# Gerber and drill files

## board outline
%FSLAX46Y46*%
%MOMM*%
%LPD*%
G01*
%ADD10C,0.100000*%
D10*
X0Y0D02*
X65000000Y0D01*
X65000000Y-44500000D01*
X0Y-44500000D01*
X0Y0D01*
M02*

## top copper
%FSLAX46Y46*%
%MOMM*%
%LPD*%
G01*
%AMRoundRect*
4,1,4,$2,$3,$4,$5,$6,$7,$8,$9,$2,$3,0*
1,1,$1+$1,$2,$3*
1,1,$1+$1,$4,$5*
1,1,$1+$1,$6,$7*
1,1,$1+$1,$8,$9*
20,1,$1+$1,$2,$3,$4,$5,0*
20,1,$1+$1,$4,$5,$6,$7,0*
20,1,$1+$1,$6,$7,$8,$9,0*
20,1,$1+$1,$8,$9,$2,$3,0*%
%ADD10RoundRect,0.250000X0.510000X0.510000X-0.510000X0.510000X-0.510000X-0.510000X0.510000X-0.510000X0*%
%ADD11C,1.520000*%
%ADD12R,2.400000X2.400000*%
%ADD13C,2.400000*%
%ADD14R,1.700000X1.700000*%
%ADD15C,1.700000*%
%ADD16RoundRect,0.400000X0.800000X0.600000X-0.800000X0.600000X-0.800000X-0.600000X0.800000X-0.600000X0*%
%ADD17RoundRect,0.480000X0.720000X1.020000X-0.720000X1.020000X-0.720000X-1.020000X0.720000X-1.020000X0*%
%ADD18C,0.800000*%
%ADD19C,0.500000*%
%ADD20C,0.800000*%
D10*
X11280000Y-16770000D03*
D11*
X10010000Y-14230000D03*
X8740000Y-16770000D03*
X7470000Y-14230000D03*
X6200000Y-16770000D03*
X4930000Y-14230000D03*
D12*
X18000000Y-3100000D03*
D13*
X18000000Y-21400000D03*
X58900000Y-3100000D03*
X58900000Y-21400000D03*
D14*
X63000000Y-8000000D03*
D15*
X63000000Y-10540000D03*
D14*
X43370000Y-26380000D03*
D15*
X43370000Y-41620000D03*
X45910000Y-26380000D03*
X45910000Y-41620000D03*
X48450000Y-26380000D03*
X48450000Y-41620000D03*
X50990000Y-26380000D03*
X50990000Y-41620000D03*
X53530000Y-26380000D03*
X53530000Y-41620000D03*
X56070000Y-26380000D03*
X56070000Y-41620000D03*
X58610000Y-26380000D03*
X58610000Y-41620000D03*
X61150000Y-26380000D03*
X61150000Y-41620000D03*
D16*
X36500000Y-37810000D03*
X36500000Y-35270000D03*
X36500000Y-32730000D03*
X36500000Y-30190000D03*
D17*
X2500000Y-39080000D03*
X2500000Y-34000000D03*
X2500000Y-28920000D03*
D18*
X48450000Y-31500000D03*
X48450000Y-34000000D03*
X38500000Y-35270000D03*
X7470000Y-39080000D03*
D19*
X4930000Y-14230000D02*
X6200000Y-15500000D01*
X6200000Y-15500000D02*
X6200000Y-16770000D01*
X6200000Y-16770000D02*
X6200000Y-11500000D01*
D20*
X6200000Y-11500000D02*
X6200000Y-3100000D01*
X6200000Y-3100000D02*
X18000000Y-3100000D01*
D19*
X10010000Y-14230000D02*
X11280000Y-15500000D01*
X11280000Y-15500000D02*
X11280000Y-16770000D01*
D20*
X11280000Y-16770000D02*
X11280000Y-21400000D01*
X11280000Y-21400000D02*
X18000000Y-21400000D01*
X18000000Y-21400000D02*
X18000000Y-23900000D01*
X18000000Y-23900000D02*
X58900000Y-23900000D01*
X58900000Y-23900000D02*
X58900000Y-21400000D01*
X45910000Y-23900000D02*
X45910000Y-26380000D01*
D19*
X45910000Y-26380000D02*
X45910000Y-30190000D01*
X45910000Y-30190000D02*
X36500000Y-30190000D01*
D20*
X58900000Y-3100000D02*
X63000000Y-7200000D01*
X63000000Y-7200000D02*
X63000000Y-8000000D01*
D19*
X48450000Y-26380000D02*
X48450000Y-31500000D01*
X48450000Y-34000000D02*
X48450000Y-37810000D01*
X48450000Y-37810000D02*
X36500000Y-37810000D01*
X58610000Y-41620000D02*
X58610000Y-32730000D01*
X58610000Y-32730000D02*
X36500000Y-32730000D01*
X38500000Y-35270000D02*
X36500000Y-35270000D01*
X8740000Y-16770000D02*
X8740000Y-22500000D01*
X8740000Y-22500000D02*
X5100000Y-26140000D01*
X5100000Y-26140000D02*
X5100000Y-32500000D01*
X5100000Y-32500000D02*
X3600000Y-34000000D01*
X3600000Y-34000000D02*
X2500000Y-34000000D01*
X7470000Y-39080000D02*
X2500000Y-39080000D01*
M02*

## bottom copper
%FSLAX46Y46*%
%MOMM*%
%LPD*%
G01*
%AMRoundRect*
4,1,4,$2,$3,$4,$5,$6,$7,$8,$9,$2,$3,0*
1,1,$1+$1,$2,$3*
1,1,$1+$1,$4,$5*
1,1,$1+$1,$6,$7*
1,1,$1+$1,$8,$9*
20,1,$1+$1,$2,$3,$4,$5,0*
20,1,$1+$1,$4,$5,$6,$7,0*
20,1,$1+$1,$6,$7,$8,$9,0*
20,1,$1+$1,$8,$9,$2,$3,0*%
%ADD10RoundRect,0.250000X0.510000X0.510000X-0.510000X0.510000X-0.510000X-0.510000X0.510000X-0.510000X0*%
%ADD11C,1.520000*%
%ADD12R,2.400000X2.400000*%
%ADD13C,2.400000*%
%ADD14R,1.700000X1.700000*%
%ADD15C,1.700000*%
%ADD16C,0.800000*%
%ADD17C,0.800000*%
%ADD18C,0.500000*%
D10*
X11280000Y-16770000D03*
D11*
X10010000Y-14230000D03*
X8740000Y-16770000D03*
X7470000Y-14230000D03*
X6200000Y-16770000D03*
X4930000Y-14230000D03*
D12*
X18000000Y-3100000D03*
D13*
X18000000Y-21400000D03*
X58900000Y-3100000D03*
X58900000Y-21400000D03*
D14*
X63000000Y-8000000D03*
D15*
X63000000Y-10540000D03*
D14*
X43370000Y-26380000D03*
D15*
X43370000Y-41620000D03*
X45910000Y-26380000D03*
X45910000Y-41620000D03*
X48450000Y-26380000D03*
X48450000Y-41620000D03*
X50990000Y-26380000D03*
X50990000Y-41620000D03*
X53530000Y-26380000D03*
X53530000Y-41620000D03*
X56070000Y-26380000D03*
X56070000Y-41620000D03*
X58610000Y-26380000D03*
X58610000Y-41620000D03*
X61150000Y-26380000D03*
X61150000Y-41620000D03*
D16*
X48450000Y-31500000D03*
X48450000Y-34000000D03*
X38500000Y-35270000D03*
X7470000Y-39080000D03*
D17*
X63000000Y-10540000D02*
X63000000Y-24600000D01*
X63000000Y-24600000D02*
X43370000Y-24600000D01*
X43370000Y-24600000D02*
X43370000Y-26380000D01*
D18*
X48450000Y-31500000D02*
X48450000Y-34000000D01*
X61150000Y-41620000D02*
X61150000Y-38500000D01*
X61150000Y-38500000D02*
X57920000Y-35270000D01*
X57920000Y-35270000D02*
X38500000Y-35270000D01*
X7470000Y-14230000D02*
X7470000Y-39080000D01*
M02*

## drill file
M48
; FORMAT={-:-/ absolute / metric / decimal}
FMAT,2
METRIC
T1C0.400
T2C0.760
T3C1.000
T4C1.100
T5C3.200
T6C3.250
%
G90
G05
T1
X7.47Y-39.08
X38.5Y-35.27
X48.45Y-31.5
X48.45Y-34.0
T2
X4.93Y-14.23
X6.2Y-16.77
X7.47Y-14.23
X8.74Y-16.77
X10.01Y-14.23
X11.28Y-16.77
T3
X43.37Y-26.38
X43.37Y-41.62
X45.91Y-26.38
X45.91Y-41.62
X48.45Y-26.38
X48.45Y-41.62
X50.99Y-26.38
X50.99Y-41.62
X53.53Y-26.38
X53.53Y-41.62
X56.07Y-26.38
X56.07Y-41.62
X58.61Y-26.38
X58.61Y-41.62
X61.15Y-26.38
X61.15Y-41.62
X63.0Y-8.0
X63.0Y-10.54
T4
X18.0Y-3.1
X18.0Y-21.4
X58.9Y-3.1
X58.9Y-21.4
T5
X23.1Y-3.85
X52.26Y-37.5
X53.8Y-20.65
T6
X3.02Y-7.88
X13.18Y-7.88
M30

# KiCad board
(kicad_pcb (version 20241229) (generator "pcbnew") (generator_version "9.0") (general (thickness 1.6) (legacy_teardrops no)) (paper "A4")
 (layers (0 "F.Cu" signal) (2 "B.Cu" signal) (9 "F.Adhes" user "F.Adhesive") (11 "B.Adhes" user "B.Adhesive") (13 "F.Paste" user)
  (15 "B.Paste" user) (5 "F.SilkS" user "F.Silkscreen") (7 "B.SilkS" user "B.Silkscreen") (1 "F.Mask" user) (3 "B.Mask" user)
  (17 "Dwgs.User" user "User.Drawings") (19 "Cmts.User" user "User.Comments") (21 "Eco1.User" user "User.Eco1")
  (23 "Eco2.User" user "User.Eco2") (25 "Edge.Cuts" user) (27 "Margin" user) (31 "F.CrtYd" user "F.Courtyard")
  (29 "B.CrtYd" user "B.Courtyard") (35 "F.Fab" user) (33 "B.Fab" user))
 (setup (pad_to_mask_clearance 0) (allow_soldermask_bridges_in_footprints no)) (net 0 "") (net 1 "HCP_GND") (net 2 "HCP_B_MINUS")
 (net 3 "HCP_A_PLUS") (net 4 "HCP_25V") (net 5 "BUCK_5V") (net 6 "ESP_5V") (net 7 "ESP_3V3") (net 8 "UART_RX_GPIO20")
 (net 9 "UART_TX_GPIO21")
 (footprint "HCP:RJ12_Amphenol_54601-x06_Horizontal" (layer "F.Cu") (at 11.28 16.77 180)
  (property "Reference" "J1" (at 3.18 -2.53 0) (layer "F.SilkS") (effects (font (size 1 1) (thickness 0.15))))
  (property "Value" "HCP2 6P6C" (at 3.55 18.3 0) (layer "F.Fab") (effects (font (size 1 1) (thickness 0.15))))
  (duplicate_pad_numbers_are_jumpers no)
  (pad "" np_thru_hole circle (at -1.9 8.89 180) (size 3.25 3.25) (drill 3.25) (layers "*.Cu" "*.Mask"))
  (pad "" np_thru_hole circle (at 8.26 8.89 180) (size 3.25 3.25) (drill 3.25) (layers "*.Cu" "*.Mask"))
  (pad "1" thru_hole roundrect (at 0 0 180) (size 1.52 1.52) (drill 0.76) (layers "*.Cu" "*.Mask") (remove_unused_layers no)
   (roundrect_rratio 0.1644736842) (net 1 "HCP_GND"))
  (pad "2" thru_hole circle (at 1.27 2.54 180) (size 1.52 1.52) (drill 0.76) (layers "*.Cu" "*.Mask") (remove_unused_layers no)
   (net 1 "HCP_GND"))
  (pad "3" thru_hole circle (at 2.54 0 180) (size 1.52 1.52) (drill 0.76) (layers "*.Cu" "*.Mask") (remove_unused_layers no)
   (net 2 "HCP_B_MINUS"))
  (pad "4" thru_hole circle (at 3.81 2.54 180) (size 1.52 1.52) (drill 0.76) (layers "*.Cu" "*.Mask") (remove_unused_layers no)
   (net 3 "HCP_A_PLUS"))
  (pad "5" thru_hole circle (at 5.08 0 180) (size 1.52 1.52) (drill 0.76) (layers "*.Cu" "*.Mask") (remove_unused_layers no)
   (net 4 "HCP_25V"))
  (pad "6" thru_hole circle (at 6.35 2.54 180) (size 1.52 1.52) (drill 0.76) (layers "*.Cu" "*.Mask") (remove_unused_layers no)
   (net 4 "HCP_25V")))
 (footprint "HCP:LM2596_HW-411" (layer "F.Cu") (at 38.45 12.25 0)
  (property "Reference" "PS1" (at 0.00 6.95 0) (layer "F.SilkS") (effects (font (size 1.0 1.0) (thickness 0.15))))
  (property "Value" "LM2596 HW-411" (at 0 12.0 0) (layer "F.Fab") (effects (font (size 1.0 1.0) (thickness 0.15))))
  (pad "1" thru_hole rect (at -20.45 -9.15) (size 2.4 2.4) (drill 1.1) (layers "*.Cu" "*.Mask") (remove_unused_layers no) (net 4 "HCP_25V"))
  (pad "2" thru_hole circle (at -20.45 9.15) (size 2.4 2.4) (drill 1.1) (layers "*.Cu" "*.Mask") (remove_unused_layers no) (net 1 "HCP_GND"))
  (pad "3" thru_hole circle (at 20.45 -9.15) (size 2.4 2.4) (drill 1.1) (layers "*.Cu" "*.Mask") (remove_unused_layers no) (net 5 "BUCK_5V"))
  (pad "4" thru_hole circle (at 20.45 9.15) (size 2.4 2.4) (drill 1.1) (layers "*.Cu" "*.Mask") (remove_unused_layers no) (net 1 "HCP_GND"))
  (pad "" np_thru_hole circle (at -15.35 -8.4) (size 3.2 3.2) (drill 3.2) (layers "*.Cu" "*.Mask"))
  (pad "" np_thru_hole circle (at 15.35 8.4) (size 3.2 3.2) (drill 3.2) (layers "*.Cu" "*.Mask")))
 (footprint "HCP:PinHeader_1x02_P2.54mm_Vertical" (layer "F.Cu") (at 63.0 8.0 0)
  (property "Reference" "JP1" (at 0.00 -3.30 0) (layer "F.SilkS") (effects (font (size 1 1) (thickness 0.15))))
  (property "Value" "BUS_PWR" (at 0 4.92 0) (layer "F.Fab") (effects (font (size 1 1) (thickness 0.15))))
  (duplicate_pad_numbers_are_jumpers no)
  (pad "1" thru_hole rect (at 0 0) (size 1.7 1.7) (drill 1) (layers "*.Cu" "*.Mask") (remove_unused_layers no) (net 5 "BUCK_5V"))
  (pad "2" thru_hole circle (at 0 2.54) (size 1.7 1.7) (drill 1) (layers "*.Cu" "*.Mask") (remove_unused_layers no) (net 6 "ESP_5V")))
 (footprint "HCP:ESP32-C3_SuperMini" (layer "F.Cu") (at 52.26 34.0 90)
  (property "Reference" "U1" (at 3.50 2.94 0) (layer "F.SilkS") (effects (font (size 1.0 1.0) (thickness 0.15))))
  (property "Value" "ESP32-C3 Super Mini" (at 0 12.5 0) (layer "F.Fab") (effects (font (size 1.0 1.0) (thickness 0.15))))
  (pad "1" thru_hole rect (at 7.62 -8.89 90) (size 1.7 1.7) (drill 1.0) (layers "*.Cu" "*.Mask") (remove_unused_layers no) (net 6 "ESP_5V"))
  (pad "2" thru_hole circle (at -7.62 -8.89 90) (size 1.7 1.7) (drill 1.0) (layers "*.Cu" "*.Mask") (remove_unused_layers no))
  (pad "3" thru_hole circle (at 7.62 -6.35 90) (size 1.7 1.7) (drill 1.0) (layers "*.Cu" "*.Mask") (remove_unused_layers no)
   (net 1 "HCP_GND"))
  (pad "4" thru_hole circle (at -7.62 -6.35 90) (size 1.7 1.7) (drill 1.0) (layers "*.Cu" "*.Mask") (remove_unused_layers no))
  (pad "5" thru_hole circle (at 7.62 -3.81 90) (size 1.7 1.7) (drill 1.0) (layers "*.Cu" "*.Mask") (remove_unused_layers no)
   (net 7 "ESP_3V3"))
  (pad "6" thru_hole circle (at -7.62 -3.81 90) (size 1.7 1.7) (drill 1.0) (layers "*.Cu" "*.Mask") (remove_unused_layers no))
  (pad "7" thru_hole circle (at 7.62 -1.27 90) (size 1.7 1.7) (drill 1.0) (layers "*.Cu" "*.Mask") (remove_unused_layers no))
  (pad "8" thru_hole circle (at -7.62 -1.27 90) (size 1.7 1.7) (drill 1.0) (layers "*.Cu" "*.Mask") (remove_unused_layers no))
  (pad "9" thru_hole circle (at 7.62 1.27 90) (size 1.7 1.7) (drill 1.0) (layers "*.Cu" "*.Mask") (remove_unused_layers no))
  (pad "10" thru_hole circle (at -7.62 1.27 90) (size 1.7 1.7) (drill 1.0) (layers "*.Cu" "*.Mask") (remove_unused_layers no))
  (pad "11" thru_hole circle (at 7.62 3.81 90) (size 1.7 1.7) (drill 1.0) (layers "*.Cu" "*.Mask") (remove_unused_layers no))
  (pad "12" thru_hole circle (at -7.62 3.81 90) (size 1.7 1.7) (drill 1.0) (layers "*.Cu" "*.Mask") (remove_unused_layers no))
  (pad "13" thru_hole circle (at 7.62 6.35 90) (size 1.7 1.7) (drill 1.0) (layers "*.Cu" "*.Mask") (remove_unused_layers no))
  (pad "14" thru_hole circle (at -7.62 6.35 90) (size 1.7 1.7) (drill 1.0) (layers "*.Cu" "*.Mask") (remove_unused_layers no)
   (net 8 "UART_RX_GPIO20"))
  (pad "15" thru_hole circle (at 7.62 8.89 90) (size 1.7 1.7) (drill 1.0) (layers "*.Cu" "*.Mask") (remove_unused_layers no))
  (pad "16" thru_hole circle (at -7.62 8.89 90) (size 1.7 1.7) (drill 1.0) (layers "*.Cu" "*.Mask") (remove_unused_layers no)
   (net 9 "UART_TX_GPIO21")))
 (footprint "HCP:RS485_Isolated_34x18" (layer "F.Cu") (at 19.5 34.0 180)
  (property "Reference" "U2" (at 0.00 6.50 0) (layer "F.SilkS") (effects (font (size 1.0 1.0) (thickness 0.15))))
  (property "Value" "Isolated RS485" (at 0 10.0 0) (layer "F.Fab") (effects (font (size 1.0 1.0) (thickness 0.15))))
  (pad "1" smd roundrect (at -17 -3.81 180) (size 2.4 2.0) (layers "F.Cu" "F.Paste" "F.Mask") (roundrect_rratio 0.2) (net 7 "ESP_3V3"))
  (pad "2" smd roundrect (at -17 -1.27 180) (size 2.4 2.0) (layers "F.Cu" "F.Paste" "F.Mask") (roundrect_rratio 0.2)
   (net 9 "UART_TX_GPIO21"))
  (pad "3" smd roundrect (at -17 1.27 180) (size 2.4 2.0) (layers "F.Cu" "F.Paste" "F.Mask") (roundrect_rratio 0.2) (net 8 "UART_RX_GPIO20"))
  (pad "4" smd roundrect (at -17 3.81 180) (size 2.4 2.0) (layers "F.Cu" "F.Paste" "F.Mask") (roundrect_rratio 0.2) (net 1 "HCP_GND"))
  (pad "5" smd roundrect (at 17 -5.08 180) (size 2.4 3.0) (layers "F.Cu" "F.Paste" "F.Mask") (roundrect_rratio 0.2) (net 3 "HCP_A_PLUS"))
  (pad "6" smd roundrect (at 17 0 180) (size 2.4 3.0) (layers "F.Cu" "F.Paste" "F.Mask") (roundrect_rratio 0.2) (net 2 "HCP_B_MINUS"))
  (pad "7" smd roundrect (at 17 5.08 180) (size 2.4 3.0) (layers "F.Cu" "F.Paste" "F.Mask") (roundrect_rratio 0.2)))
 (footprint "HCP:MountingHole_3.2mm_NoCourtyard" (layer "F.Cu") (at 52.26 37.5 0)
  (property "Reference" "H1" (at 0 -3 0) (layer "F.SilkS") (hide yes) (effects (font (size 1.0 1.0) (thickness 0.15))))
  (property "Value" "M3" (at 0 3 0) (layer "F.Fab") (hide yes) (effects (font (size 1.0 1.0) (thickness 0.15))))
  (pad "" np_thru_hole circle (at 0 0) (size 3.2 3.2) (drill 3.2) (layers "*.Cu" "*.Mask")))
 (segment (start 4.93 14.23) (end 6.2 15.5) (width 0.5) (layer "F.Cu") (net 4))
 (segment (start 6.2 15.5) (end 6.2 16.77) (width 0.5) (layer "F.Cu") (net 4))
 (segment (start 6.2 16.77) (end 6.2 11.5) (width 0.5) (layer "F.Cu") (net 4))
 (segment (start 6.2 11.5) (end 6.2 3.1) (width 0.8) (layer "F.Cu") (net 4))
 (segment (start 6.2 3.1) (end 18.0 3.1) (width 0.8) (layer "F.Cu") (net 4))
 (segment (start 10.01 14.23) (end 11.28 15.5) (width 0.5) (layer "F.Cu") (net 1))
 (segment (start 11.28 15.5) (end 11.28 16.77) (width 0.5) (layer "F.Cu") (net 1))
 (segment (start 11.28 16.77) (end 11.28 21.4) (width 0.8) (layer "F.Cu") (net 1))
 (segment (start 11.28 21.4) (end 18.0 21.4) (width 0.8) (layer "F.Cu") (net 1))
 (segment (start 18.0 21.4) (end 18.0 23.9) (width 0.8) (layer "F.Cu") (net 1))
 (segment (start 18.0 23.9) (end 58.9 23.9) (width 0.8) (layer "F.Cu") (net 1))
 (segment (start 58.9 23.9) (end 58.9 21.4) (width 0.8) (layer "F.Cu") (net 1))
 (segment (start 45.91 23.9) (end 45.91 26.38) (width 0.8) (layer "F.Cu") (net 1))
 (segment (start 45.91 26.38) (end 45.91 30.19) (width 0.5) (layer "F.Cu") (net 1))
 (segment (start 45.91 30.19) (end 36.5 30.19) (width 0.5) (layer "F.Cu") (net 1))
 (segment (start 58.9 3.1) (end 63.0 7.2) (width 0.8) (layer "F.Cu") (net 5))
 (segment (start 63.0 7.2) (end 63.0 8.0) (width 0.8) (layer "F.Cu") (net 5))
 (segment (start 63.0 10.54) (end 63.0 24.6) (width 0.8) (layer "B.Cu") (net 6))
 (segment (start 63.0 24.6) (end 43.37 24.6) (width 0.8) (layer "B.Cu") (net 6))
 (segment (start 43.37 24.6) (end 43.37 26.38) (width 0.8) (layer "B.Cu") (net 6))
 (segment (start 48.45 26.38) (end 48.45 31.5) (width 0.5) (layer "F.Cu") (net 7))
 (segment (start 48.45 31.5) (end 48.45 34.0) (width 0.5) (layer "B.Cu") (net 7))
 (segment (start 48.45 34.0) (end 48.45 37.81) (width 0.5) (layer "F.Cu") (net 7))
 (segment (start 48.45 37.81) (end 36.5 37.81) (width 0.5) (layer "F.Cu") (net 7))
 (segment (start 58.61 41.62) (end 58.61 32.73) (width 0.5) (layer "F.Cu") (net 8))
 (segment (start 58.61 32.73) (end 36.5 32.73) (width 0.5) (layer "F.Cu") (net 8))
 (segment (start 61.15 41.62) (end 61.15 38.5) (width 0.5) (layer "B.Cu") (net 9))
 (segment (start 61.15 38.5) (end 57.92 35.27) (width 0.5) (layer "B.Cu") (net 9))
 (segment (start 57.92 35.27) (end 38.5 35.27) (width 0.5) (layer "B.Cu") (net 9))
 (segment (start 38.5 35.27) (end 36.5 35.27) (width 0.5) (layer "F.Cu") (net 9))
 (segment (start 8.74 16.77) (end 8.74 22.5) (width 0.5) (layer "F.Cu") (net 2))
 (segment (start 8.74 22.5) (end 5.1 26.14) (width 0.5) (layer "F.Cu") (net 2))
 (segment (start 5.1 26.14) (end 5.1 32.5) (width 0.5) (layer "F.Cu") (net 2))
 (segment (start 5.1 32.5) (end 3.6 34.0) (width 0.5) (layer "F.Cu") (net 2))
 (segment (start 3.6 34.0) (end 2.5 34.0) (width 0.5) (layer "F.Cu") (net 2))
 (segment (start 7.47 14.23) (end 7.47 39.08) (width 0.5) (layer "B.Cu") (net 3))
 (segment (start 7.47 39.08) (end 2.5 39.08) (width 0.5) (layer "F.Cu") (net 3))
 (via (at 48.45 31.5) (size 0.8) (drill 0.4) (layers "F.Cu" "B.Cu") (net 7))
 (via (at 48.45 34.0) (size 0.8) (drill 0.4) (layers "F.Cu" "B.Cu") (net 7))
 (via (at 38.5 35.27) (size 0.8) (drill 0.4) (layers "F.Cu" "B.Cu") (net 9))
 (via (at 7.47 39.08) (size 0.8) (drill 0.4) (layers "F.Cu" "B.Cu") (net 3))
 (gr_rect (start 0 0) (end 65.0 44.5) (stroke (width 0.1) (type default)) (fill none) (layer "Edge.Cuts")))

